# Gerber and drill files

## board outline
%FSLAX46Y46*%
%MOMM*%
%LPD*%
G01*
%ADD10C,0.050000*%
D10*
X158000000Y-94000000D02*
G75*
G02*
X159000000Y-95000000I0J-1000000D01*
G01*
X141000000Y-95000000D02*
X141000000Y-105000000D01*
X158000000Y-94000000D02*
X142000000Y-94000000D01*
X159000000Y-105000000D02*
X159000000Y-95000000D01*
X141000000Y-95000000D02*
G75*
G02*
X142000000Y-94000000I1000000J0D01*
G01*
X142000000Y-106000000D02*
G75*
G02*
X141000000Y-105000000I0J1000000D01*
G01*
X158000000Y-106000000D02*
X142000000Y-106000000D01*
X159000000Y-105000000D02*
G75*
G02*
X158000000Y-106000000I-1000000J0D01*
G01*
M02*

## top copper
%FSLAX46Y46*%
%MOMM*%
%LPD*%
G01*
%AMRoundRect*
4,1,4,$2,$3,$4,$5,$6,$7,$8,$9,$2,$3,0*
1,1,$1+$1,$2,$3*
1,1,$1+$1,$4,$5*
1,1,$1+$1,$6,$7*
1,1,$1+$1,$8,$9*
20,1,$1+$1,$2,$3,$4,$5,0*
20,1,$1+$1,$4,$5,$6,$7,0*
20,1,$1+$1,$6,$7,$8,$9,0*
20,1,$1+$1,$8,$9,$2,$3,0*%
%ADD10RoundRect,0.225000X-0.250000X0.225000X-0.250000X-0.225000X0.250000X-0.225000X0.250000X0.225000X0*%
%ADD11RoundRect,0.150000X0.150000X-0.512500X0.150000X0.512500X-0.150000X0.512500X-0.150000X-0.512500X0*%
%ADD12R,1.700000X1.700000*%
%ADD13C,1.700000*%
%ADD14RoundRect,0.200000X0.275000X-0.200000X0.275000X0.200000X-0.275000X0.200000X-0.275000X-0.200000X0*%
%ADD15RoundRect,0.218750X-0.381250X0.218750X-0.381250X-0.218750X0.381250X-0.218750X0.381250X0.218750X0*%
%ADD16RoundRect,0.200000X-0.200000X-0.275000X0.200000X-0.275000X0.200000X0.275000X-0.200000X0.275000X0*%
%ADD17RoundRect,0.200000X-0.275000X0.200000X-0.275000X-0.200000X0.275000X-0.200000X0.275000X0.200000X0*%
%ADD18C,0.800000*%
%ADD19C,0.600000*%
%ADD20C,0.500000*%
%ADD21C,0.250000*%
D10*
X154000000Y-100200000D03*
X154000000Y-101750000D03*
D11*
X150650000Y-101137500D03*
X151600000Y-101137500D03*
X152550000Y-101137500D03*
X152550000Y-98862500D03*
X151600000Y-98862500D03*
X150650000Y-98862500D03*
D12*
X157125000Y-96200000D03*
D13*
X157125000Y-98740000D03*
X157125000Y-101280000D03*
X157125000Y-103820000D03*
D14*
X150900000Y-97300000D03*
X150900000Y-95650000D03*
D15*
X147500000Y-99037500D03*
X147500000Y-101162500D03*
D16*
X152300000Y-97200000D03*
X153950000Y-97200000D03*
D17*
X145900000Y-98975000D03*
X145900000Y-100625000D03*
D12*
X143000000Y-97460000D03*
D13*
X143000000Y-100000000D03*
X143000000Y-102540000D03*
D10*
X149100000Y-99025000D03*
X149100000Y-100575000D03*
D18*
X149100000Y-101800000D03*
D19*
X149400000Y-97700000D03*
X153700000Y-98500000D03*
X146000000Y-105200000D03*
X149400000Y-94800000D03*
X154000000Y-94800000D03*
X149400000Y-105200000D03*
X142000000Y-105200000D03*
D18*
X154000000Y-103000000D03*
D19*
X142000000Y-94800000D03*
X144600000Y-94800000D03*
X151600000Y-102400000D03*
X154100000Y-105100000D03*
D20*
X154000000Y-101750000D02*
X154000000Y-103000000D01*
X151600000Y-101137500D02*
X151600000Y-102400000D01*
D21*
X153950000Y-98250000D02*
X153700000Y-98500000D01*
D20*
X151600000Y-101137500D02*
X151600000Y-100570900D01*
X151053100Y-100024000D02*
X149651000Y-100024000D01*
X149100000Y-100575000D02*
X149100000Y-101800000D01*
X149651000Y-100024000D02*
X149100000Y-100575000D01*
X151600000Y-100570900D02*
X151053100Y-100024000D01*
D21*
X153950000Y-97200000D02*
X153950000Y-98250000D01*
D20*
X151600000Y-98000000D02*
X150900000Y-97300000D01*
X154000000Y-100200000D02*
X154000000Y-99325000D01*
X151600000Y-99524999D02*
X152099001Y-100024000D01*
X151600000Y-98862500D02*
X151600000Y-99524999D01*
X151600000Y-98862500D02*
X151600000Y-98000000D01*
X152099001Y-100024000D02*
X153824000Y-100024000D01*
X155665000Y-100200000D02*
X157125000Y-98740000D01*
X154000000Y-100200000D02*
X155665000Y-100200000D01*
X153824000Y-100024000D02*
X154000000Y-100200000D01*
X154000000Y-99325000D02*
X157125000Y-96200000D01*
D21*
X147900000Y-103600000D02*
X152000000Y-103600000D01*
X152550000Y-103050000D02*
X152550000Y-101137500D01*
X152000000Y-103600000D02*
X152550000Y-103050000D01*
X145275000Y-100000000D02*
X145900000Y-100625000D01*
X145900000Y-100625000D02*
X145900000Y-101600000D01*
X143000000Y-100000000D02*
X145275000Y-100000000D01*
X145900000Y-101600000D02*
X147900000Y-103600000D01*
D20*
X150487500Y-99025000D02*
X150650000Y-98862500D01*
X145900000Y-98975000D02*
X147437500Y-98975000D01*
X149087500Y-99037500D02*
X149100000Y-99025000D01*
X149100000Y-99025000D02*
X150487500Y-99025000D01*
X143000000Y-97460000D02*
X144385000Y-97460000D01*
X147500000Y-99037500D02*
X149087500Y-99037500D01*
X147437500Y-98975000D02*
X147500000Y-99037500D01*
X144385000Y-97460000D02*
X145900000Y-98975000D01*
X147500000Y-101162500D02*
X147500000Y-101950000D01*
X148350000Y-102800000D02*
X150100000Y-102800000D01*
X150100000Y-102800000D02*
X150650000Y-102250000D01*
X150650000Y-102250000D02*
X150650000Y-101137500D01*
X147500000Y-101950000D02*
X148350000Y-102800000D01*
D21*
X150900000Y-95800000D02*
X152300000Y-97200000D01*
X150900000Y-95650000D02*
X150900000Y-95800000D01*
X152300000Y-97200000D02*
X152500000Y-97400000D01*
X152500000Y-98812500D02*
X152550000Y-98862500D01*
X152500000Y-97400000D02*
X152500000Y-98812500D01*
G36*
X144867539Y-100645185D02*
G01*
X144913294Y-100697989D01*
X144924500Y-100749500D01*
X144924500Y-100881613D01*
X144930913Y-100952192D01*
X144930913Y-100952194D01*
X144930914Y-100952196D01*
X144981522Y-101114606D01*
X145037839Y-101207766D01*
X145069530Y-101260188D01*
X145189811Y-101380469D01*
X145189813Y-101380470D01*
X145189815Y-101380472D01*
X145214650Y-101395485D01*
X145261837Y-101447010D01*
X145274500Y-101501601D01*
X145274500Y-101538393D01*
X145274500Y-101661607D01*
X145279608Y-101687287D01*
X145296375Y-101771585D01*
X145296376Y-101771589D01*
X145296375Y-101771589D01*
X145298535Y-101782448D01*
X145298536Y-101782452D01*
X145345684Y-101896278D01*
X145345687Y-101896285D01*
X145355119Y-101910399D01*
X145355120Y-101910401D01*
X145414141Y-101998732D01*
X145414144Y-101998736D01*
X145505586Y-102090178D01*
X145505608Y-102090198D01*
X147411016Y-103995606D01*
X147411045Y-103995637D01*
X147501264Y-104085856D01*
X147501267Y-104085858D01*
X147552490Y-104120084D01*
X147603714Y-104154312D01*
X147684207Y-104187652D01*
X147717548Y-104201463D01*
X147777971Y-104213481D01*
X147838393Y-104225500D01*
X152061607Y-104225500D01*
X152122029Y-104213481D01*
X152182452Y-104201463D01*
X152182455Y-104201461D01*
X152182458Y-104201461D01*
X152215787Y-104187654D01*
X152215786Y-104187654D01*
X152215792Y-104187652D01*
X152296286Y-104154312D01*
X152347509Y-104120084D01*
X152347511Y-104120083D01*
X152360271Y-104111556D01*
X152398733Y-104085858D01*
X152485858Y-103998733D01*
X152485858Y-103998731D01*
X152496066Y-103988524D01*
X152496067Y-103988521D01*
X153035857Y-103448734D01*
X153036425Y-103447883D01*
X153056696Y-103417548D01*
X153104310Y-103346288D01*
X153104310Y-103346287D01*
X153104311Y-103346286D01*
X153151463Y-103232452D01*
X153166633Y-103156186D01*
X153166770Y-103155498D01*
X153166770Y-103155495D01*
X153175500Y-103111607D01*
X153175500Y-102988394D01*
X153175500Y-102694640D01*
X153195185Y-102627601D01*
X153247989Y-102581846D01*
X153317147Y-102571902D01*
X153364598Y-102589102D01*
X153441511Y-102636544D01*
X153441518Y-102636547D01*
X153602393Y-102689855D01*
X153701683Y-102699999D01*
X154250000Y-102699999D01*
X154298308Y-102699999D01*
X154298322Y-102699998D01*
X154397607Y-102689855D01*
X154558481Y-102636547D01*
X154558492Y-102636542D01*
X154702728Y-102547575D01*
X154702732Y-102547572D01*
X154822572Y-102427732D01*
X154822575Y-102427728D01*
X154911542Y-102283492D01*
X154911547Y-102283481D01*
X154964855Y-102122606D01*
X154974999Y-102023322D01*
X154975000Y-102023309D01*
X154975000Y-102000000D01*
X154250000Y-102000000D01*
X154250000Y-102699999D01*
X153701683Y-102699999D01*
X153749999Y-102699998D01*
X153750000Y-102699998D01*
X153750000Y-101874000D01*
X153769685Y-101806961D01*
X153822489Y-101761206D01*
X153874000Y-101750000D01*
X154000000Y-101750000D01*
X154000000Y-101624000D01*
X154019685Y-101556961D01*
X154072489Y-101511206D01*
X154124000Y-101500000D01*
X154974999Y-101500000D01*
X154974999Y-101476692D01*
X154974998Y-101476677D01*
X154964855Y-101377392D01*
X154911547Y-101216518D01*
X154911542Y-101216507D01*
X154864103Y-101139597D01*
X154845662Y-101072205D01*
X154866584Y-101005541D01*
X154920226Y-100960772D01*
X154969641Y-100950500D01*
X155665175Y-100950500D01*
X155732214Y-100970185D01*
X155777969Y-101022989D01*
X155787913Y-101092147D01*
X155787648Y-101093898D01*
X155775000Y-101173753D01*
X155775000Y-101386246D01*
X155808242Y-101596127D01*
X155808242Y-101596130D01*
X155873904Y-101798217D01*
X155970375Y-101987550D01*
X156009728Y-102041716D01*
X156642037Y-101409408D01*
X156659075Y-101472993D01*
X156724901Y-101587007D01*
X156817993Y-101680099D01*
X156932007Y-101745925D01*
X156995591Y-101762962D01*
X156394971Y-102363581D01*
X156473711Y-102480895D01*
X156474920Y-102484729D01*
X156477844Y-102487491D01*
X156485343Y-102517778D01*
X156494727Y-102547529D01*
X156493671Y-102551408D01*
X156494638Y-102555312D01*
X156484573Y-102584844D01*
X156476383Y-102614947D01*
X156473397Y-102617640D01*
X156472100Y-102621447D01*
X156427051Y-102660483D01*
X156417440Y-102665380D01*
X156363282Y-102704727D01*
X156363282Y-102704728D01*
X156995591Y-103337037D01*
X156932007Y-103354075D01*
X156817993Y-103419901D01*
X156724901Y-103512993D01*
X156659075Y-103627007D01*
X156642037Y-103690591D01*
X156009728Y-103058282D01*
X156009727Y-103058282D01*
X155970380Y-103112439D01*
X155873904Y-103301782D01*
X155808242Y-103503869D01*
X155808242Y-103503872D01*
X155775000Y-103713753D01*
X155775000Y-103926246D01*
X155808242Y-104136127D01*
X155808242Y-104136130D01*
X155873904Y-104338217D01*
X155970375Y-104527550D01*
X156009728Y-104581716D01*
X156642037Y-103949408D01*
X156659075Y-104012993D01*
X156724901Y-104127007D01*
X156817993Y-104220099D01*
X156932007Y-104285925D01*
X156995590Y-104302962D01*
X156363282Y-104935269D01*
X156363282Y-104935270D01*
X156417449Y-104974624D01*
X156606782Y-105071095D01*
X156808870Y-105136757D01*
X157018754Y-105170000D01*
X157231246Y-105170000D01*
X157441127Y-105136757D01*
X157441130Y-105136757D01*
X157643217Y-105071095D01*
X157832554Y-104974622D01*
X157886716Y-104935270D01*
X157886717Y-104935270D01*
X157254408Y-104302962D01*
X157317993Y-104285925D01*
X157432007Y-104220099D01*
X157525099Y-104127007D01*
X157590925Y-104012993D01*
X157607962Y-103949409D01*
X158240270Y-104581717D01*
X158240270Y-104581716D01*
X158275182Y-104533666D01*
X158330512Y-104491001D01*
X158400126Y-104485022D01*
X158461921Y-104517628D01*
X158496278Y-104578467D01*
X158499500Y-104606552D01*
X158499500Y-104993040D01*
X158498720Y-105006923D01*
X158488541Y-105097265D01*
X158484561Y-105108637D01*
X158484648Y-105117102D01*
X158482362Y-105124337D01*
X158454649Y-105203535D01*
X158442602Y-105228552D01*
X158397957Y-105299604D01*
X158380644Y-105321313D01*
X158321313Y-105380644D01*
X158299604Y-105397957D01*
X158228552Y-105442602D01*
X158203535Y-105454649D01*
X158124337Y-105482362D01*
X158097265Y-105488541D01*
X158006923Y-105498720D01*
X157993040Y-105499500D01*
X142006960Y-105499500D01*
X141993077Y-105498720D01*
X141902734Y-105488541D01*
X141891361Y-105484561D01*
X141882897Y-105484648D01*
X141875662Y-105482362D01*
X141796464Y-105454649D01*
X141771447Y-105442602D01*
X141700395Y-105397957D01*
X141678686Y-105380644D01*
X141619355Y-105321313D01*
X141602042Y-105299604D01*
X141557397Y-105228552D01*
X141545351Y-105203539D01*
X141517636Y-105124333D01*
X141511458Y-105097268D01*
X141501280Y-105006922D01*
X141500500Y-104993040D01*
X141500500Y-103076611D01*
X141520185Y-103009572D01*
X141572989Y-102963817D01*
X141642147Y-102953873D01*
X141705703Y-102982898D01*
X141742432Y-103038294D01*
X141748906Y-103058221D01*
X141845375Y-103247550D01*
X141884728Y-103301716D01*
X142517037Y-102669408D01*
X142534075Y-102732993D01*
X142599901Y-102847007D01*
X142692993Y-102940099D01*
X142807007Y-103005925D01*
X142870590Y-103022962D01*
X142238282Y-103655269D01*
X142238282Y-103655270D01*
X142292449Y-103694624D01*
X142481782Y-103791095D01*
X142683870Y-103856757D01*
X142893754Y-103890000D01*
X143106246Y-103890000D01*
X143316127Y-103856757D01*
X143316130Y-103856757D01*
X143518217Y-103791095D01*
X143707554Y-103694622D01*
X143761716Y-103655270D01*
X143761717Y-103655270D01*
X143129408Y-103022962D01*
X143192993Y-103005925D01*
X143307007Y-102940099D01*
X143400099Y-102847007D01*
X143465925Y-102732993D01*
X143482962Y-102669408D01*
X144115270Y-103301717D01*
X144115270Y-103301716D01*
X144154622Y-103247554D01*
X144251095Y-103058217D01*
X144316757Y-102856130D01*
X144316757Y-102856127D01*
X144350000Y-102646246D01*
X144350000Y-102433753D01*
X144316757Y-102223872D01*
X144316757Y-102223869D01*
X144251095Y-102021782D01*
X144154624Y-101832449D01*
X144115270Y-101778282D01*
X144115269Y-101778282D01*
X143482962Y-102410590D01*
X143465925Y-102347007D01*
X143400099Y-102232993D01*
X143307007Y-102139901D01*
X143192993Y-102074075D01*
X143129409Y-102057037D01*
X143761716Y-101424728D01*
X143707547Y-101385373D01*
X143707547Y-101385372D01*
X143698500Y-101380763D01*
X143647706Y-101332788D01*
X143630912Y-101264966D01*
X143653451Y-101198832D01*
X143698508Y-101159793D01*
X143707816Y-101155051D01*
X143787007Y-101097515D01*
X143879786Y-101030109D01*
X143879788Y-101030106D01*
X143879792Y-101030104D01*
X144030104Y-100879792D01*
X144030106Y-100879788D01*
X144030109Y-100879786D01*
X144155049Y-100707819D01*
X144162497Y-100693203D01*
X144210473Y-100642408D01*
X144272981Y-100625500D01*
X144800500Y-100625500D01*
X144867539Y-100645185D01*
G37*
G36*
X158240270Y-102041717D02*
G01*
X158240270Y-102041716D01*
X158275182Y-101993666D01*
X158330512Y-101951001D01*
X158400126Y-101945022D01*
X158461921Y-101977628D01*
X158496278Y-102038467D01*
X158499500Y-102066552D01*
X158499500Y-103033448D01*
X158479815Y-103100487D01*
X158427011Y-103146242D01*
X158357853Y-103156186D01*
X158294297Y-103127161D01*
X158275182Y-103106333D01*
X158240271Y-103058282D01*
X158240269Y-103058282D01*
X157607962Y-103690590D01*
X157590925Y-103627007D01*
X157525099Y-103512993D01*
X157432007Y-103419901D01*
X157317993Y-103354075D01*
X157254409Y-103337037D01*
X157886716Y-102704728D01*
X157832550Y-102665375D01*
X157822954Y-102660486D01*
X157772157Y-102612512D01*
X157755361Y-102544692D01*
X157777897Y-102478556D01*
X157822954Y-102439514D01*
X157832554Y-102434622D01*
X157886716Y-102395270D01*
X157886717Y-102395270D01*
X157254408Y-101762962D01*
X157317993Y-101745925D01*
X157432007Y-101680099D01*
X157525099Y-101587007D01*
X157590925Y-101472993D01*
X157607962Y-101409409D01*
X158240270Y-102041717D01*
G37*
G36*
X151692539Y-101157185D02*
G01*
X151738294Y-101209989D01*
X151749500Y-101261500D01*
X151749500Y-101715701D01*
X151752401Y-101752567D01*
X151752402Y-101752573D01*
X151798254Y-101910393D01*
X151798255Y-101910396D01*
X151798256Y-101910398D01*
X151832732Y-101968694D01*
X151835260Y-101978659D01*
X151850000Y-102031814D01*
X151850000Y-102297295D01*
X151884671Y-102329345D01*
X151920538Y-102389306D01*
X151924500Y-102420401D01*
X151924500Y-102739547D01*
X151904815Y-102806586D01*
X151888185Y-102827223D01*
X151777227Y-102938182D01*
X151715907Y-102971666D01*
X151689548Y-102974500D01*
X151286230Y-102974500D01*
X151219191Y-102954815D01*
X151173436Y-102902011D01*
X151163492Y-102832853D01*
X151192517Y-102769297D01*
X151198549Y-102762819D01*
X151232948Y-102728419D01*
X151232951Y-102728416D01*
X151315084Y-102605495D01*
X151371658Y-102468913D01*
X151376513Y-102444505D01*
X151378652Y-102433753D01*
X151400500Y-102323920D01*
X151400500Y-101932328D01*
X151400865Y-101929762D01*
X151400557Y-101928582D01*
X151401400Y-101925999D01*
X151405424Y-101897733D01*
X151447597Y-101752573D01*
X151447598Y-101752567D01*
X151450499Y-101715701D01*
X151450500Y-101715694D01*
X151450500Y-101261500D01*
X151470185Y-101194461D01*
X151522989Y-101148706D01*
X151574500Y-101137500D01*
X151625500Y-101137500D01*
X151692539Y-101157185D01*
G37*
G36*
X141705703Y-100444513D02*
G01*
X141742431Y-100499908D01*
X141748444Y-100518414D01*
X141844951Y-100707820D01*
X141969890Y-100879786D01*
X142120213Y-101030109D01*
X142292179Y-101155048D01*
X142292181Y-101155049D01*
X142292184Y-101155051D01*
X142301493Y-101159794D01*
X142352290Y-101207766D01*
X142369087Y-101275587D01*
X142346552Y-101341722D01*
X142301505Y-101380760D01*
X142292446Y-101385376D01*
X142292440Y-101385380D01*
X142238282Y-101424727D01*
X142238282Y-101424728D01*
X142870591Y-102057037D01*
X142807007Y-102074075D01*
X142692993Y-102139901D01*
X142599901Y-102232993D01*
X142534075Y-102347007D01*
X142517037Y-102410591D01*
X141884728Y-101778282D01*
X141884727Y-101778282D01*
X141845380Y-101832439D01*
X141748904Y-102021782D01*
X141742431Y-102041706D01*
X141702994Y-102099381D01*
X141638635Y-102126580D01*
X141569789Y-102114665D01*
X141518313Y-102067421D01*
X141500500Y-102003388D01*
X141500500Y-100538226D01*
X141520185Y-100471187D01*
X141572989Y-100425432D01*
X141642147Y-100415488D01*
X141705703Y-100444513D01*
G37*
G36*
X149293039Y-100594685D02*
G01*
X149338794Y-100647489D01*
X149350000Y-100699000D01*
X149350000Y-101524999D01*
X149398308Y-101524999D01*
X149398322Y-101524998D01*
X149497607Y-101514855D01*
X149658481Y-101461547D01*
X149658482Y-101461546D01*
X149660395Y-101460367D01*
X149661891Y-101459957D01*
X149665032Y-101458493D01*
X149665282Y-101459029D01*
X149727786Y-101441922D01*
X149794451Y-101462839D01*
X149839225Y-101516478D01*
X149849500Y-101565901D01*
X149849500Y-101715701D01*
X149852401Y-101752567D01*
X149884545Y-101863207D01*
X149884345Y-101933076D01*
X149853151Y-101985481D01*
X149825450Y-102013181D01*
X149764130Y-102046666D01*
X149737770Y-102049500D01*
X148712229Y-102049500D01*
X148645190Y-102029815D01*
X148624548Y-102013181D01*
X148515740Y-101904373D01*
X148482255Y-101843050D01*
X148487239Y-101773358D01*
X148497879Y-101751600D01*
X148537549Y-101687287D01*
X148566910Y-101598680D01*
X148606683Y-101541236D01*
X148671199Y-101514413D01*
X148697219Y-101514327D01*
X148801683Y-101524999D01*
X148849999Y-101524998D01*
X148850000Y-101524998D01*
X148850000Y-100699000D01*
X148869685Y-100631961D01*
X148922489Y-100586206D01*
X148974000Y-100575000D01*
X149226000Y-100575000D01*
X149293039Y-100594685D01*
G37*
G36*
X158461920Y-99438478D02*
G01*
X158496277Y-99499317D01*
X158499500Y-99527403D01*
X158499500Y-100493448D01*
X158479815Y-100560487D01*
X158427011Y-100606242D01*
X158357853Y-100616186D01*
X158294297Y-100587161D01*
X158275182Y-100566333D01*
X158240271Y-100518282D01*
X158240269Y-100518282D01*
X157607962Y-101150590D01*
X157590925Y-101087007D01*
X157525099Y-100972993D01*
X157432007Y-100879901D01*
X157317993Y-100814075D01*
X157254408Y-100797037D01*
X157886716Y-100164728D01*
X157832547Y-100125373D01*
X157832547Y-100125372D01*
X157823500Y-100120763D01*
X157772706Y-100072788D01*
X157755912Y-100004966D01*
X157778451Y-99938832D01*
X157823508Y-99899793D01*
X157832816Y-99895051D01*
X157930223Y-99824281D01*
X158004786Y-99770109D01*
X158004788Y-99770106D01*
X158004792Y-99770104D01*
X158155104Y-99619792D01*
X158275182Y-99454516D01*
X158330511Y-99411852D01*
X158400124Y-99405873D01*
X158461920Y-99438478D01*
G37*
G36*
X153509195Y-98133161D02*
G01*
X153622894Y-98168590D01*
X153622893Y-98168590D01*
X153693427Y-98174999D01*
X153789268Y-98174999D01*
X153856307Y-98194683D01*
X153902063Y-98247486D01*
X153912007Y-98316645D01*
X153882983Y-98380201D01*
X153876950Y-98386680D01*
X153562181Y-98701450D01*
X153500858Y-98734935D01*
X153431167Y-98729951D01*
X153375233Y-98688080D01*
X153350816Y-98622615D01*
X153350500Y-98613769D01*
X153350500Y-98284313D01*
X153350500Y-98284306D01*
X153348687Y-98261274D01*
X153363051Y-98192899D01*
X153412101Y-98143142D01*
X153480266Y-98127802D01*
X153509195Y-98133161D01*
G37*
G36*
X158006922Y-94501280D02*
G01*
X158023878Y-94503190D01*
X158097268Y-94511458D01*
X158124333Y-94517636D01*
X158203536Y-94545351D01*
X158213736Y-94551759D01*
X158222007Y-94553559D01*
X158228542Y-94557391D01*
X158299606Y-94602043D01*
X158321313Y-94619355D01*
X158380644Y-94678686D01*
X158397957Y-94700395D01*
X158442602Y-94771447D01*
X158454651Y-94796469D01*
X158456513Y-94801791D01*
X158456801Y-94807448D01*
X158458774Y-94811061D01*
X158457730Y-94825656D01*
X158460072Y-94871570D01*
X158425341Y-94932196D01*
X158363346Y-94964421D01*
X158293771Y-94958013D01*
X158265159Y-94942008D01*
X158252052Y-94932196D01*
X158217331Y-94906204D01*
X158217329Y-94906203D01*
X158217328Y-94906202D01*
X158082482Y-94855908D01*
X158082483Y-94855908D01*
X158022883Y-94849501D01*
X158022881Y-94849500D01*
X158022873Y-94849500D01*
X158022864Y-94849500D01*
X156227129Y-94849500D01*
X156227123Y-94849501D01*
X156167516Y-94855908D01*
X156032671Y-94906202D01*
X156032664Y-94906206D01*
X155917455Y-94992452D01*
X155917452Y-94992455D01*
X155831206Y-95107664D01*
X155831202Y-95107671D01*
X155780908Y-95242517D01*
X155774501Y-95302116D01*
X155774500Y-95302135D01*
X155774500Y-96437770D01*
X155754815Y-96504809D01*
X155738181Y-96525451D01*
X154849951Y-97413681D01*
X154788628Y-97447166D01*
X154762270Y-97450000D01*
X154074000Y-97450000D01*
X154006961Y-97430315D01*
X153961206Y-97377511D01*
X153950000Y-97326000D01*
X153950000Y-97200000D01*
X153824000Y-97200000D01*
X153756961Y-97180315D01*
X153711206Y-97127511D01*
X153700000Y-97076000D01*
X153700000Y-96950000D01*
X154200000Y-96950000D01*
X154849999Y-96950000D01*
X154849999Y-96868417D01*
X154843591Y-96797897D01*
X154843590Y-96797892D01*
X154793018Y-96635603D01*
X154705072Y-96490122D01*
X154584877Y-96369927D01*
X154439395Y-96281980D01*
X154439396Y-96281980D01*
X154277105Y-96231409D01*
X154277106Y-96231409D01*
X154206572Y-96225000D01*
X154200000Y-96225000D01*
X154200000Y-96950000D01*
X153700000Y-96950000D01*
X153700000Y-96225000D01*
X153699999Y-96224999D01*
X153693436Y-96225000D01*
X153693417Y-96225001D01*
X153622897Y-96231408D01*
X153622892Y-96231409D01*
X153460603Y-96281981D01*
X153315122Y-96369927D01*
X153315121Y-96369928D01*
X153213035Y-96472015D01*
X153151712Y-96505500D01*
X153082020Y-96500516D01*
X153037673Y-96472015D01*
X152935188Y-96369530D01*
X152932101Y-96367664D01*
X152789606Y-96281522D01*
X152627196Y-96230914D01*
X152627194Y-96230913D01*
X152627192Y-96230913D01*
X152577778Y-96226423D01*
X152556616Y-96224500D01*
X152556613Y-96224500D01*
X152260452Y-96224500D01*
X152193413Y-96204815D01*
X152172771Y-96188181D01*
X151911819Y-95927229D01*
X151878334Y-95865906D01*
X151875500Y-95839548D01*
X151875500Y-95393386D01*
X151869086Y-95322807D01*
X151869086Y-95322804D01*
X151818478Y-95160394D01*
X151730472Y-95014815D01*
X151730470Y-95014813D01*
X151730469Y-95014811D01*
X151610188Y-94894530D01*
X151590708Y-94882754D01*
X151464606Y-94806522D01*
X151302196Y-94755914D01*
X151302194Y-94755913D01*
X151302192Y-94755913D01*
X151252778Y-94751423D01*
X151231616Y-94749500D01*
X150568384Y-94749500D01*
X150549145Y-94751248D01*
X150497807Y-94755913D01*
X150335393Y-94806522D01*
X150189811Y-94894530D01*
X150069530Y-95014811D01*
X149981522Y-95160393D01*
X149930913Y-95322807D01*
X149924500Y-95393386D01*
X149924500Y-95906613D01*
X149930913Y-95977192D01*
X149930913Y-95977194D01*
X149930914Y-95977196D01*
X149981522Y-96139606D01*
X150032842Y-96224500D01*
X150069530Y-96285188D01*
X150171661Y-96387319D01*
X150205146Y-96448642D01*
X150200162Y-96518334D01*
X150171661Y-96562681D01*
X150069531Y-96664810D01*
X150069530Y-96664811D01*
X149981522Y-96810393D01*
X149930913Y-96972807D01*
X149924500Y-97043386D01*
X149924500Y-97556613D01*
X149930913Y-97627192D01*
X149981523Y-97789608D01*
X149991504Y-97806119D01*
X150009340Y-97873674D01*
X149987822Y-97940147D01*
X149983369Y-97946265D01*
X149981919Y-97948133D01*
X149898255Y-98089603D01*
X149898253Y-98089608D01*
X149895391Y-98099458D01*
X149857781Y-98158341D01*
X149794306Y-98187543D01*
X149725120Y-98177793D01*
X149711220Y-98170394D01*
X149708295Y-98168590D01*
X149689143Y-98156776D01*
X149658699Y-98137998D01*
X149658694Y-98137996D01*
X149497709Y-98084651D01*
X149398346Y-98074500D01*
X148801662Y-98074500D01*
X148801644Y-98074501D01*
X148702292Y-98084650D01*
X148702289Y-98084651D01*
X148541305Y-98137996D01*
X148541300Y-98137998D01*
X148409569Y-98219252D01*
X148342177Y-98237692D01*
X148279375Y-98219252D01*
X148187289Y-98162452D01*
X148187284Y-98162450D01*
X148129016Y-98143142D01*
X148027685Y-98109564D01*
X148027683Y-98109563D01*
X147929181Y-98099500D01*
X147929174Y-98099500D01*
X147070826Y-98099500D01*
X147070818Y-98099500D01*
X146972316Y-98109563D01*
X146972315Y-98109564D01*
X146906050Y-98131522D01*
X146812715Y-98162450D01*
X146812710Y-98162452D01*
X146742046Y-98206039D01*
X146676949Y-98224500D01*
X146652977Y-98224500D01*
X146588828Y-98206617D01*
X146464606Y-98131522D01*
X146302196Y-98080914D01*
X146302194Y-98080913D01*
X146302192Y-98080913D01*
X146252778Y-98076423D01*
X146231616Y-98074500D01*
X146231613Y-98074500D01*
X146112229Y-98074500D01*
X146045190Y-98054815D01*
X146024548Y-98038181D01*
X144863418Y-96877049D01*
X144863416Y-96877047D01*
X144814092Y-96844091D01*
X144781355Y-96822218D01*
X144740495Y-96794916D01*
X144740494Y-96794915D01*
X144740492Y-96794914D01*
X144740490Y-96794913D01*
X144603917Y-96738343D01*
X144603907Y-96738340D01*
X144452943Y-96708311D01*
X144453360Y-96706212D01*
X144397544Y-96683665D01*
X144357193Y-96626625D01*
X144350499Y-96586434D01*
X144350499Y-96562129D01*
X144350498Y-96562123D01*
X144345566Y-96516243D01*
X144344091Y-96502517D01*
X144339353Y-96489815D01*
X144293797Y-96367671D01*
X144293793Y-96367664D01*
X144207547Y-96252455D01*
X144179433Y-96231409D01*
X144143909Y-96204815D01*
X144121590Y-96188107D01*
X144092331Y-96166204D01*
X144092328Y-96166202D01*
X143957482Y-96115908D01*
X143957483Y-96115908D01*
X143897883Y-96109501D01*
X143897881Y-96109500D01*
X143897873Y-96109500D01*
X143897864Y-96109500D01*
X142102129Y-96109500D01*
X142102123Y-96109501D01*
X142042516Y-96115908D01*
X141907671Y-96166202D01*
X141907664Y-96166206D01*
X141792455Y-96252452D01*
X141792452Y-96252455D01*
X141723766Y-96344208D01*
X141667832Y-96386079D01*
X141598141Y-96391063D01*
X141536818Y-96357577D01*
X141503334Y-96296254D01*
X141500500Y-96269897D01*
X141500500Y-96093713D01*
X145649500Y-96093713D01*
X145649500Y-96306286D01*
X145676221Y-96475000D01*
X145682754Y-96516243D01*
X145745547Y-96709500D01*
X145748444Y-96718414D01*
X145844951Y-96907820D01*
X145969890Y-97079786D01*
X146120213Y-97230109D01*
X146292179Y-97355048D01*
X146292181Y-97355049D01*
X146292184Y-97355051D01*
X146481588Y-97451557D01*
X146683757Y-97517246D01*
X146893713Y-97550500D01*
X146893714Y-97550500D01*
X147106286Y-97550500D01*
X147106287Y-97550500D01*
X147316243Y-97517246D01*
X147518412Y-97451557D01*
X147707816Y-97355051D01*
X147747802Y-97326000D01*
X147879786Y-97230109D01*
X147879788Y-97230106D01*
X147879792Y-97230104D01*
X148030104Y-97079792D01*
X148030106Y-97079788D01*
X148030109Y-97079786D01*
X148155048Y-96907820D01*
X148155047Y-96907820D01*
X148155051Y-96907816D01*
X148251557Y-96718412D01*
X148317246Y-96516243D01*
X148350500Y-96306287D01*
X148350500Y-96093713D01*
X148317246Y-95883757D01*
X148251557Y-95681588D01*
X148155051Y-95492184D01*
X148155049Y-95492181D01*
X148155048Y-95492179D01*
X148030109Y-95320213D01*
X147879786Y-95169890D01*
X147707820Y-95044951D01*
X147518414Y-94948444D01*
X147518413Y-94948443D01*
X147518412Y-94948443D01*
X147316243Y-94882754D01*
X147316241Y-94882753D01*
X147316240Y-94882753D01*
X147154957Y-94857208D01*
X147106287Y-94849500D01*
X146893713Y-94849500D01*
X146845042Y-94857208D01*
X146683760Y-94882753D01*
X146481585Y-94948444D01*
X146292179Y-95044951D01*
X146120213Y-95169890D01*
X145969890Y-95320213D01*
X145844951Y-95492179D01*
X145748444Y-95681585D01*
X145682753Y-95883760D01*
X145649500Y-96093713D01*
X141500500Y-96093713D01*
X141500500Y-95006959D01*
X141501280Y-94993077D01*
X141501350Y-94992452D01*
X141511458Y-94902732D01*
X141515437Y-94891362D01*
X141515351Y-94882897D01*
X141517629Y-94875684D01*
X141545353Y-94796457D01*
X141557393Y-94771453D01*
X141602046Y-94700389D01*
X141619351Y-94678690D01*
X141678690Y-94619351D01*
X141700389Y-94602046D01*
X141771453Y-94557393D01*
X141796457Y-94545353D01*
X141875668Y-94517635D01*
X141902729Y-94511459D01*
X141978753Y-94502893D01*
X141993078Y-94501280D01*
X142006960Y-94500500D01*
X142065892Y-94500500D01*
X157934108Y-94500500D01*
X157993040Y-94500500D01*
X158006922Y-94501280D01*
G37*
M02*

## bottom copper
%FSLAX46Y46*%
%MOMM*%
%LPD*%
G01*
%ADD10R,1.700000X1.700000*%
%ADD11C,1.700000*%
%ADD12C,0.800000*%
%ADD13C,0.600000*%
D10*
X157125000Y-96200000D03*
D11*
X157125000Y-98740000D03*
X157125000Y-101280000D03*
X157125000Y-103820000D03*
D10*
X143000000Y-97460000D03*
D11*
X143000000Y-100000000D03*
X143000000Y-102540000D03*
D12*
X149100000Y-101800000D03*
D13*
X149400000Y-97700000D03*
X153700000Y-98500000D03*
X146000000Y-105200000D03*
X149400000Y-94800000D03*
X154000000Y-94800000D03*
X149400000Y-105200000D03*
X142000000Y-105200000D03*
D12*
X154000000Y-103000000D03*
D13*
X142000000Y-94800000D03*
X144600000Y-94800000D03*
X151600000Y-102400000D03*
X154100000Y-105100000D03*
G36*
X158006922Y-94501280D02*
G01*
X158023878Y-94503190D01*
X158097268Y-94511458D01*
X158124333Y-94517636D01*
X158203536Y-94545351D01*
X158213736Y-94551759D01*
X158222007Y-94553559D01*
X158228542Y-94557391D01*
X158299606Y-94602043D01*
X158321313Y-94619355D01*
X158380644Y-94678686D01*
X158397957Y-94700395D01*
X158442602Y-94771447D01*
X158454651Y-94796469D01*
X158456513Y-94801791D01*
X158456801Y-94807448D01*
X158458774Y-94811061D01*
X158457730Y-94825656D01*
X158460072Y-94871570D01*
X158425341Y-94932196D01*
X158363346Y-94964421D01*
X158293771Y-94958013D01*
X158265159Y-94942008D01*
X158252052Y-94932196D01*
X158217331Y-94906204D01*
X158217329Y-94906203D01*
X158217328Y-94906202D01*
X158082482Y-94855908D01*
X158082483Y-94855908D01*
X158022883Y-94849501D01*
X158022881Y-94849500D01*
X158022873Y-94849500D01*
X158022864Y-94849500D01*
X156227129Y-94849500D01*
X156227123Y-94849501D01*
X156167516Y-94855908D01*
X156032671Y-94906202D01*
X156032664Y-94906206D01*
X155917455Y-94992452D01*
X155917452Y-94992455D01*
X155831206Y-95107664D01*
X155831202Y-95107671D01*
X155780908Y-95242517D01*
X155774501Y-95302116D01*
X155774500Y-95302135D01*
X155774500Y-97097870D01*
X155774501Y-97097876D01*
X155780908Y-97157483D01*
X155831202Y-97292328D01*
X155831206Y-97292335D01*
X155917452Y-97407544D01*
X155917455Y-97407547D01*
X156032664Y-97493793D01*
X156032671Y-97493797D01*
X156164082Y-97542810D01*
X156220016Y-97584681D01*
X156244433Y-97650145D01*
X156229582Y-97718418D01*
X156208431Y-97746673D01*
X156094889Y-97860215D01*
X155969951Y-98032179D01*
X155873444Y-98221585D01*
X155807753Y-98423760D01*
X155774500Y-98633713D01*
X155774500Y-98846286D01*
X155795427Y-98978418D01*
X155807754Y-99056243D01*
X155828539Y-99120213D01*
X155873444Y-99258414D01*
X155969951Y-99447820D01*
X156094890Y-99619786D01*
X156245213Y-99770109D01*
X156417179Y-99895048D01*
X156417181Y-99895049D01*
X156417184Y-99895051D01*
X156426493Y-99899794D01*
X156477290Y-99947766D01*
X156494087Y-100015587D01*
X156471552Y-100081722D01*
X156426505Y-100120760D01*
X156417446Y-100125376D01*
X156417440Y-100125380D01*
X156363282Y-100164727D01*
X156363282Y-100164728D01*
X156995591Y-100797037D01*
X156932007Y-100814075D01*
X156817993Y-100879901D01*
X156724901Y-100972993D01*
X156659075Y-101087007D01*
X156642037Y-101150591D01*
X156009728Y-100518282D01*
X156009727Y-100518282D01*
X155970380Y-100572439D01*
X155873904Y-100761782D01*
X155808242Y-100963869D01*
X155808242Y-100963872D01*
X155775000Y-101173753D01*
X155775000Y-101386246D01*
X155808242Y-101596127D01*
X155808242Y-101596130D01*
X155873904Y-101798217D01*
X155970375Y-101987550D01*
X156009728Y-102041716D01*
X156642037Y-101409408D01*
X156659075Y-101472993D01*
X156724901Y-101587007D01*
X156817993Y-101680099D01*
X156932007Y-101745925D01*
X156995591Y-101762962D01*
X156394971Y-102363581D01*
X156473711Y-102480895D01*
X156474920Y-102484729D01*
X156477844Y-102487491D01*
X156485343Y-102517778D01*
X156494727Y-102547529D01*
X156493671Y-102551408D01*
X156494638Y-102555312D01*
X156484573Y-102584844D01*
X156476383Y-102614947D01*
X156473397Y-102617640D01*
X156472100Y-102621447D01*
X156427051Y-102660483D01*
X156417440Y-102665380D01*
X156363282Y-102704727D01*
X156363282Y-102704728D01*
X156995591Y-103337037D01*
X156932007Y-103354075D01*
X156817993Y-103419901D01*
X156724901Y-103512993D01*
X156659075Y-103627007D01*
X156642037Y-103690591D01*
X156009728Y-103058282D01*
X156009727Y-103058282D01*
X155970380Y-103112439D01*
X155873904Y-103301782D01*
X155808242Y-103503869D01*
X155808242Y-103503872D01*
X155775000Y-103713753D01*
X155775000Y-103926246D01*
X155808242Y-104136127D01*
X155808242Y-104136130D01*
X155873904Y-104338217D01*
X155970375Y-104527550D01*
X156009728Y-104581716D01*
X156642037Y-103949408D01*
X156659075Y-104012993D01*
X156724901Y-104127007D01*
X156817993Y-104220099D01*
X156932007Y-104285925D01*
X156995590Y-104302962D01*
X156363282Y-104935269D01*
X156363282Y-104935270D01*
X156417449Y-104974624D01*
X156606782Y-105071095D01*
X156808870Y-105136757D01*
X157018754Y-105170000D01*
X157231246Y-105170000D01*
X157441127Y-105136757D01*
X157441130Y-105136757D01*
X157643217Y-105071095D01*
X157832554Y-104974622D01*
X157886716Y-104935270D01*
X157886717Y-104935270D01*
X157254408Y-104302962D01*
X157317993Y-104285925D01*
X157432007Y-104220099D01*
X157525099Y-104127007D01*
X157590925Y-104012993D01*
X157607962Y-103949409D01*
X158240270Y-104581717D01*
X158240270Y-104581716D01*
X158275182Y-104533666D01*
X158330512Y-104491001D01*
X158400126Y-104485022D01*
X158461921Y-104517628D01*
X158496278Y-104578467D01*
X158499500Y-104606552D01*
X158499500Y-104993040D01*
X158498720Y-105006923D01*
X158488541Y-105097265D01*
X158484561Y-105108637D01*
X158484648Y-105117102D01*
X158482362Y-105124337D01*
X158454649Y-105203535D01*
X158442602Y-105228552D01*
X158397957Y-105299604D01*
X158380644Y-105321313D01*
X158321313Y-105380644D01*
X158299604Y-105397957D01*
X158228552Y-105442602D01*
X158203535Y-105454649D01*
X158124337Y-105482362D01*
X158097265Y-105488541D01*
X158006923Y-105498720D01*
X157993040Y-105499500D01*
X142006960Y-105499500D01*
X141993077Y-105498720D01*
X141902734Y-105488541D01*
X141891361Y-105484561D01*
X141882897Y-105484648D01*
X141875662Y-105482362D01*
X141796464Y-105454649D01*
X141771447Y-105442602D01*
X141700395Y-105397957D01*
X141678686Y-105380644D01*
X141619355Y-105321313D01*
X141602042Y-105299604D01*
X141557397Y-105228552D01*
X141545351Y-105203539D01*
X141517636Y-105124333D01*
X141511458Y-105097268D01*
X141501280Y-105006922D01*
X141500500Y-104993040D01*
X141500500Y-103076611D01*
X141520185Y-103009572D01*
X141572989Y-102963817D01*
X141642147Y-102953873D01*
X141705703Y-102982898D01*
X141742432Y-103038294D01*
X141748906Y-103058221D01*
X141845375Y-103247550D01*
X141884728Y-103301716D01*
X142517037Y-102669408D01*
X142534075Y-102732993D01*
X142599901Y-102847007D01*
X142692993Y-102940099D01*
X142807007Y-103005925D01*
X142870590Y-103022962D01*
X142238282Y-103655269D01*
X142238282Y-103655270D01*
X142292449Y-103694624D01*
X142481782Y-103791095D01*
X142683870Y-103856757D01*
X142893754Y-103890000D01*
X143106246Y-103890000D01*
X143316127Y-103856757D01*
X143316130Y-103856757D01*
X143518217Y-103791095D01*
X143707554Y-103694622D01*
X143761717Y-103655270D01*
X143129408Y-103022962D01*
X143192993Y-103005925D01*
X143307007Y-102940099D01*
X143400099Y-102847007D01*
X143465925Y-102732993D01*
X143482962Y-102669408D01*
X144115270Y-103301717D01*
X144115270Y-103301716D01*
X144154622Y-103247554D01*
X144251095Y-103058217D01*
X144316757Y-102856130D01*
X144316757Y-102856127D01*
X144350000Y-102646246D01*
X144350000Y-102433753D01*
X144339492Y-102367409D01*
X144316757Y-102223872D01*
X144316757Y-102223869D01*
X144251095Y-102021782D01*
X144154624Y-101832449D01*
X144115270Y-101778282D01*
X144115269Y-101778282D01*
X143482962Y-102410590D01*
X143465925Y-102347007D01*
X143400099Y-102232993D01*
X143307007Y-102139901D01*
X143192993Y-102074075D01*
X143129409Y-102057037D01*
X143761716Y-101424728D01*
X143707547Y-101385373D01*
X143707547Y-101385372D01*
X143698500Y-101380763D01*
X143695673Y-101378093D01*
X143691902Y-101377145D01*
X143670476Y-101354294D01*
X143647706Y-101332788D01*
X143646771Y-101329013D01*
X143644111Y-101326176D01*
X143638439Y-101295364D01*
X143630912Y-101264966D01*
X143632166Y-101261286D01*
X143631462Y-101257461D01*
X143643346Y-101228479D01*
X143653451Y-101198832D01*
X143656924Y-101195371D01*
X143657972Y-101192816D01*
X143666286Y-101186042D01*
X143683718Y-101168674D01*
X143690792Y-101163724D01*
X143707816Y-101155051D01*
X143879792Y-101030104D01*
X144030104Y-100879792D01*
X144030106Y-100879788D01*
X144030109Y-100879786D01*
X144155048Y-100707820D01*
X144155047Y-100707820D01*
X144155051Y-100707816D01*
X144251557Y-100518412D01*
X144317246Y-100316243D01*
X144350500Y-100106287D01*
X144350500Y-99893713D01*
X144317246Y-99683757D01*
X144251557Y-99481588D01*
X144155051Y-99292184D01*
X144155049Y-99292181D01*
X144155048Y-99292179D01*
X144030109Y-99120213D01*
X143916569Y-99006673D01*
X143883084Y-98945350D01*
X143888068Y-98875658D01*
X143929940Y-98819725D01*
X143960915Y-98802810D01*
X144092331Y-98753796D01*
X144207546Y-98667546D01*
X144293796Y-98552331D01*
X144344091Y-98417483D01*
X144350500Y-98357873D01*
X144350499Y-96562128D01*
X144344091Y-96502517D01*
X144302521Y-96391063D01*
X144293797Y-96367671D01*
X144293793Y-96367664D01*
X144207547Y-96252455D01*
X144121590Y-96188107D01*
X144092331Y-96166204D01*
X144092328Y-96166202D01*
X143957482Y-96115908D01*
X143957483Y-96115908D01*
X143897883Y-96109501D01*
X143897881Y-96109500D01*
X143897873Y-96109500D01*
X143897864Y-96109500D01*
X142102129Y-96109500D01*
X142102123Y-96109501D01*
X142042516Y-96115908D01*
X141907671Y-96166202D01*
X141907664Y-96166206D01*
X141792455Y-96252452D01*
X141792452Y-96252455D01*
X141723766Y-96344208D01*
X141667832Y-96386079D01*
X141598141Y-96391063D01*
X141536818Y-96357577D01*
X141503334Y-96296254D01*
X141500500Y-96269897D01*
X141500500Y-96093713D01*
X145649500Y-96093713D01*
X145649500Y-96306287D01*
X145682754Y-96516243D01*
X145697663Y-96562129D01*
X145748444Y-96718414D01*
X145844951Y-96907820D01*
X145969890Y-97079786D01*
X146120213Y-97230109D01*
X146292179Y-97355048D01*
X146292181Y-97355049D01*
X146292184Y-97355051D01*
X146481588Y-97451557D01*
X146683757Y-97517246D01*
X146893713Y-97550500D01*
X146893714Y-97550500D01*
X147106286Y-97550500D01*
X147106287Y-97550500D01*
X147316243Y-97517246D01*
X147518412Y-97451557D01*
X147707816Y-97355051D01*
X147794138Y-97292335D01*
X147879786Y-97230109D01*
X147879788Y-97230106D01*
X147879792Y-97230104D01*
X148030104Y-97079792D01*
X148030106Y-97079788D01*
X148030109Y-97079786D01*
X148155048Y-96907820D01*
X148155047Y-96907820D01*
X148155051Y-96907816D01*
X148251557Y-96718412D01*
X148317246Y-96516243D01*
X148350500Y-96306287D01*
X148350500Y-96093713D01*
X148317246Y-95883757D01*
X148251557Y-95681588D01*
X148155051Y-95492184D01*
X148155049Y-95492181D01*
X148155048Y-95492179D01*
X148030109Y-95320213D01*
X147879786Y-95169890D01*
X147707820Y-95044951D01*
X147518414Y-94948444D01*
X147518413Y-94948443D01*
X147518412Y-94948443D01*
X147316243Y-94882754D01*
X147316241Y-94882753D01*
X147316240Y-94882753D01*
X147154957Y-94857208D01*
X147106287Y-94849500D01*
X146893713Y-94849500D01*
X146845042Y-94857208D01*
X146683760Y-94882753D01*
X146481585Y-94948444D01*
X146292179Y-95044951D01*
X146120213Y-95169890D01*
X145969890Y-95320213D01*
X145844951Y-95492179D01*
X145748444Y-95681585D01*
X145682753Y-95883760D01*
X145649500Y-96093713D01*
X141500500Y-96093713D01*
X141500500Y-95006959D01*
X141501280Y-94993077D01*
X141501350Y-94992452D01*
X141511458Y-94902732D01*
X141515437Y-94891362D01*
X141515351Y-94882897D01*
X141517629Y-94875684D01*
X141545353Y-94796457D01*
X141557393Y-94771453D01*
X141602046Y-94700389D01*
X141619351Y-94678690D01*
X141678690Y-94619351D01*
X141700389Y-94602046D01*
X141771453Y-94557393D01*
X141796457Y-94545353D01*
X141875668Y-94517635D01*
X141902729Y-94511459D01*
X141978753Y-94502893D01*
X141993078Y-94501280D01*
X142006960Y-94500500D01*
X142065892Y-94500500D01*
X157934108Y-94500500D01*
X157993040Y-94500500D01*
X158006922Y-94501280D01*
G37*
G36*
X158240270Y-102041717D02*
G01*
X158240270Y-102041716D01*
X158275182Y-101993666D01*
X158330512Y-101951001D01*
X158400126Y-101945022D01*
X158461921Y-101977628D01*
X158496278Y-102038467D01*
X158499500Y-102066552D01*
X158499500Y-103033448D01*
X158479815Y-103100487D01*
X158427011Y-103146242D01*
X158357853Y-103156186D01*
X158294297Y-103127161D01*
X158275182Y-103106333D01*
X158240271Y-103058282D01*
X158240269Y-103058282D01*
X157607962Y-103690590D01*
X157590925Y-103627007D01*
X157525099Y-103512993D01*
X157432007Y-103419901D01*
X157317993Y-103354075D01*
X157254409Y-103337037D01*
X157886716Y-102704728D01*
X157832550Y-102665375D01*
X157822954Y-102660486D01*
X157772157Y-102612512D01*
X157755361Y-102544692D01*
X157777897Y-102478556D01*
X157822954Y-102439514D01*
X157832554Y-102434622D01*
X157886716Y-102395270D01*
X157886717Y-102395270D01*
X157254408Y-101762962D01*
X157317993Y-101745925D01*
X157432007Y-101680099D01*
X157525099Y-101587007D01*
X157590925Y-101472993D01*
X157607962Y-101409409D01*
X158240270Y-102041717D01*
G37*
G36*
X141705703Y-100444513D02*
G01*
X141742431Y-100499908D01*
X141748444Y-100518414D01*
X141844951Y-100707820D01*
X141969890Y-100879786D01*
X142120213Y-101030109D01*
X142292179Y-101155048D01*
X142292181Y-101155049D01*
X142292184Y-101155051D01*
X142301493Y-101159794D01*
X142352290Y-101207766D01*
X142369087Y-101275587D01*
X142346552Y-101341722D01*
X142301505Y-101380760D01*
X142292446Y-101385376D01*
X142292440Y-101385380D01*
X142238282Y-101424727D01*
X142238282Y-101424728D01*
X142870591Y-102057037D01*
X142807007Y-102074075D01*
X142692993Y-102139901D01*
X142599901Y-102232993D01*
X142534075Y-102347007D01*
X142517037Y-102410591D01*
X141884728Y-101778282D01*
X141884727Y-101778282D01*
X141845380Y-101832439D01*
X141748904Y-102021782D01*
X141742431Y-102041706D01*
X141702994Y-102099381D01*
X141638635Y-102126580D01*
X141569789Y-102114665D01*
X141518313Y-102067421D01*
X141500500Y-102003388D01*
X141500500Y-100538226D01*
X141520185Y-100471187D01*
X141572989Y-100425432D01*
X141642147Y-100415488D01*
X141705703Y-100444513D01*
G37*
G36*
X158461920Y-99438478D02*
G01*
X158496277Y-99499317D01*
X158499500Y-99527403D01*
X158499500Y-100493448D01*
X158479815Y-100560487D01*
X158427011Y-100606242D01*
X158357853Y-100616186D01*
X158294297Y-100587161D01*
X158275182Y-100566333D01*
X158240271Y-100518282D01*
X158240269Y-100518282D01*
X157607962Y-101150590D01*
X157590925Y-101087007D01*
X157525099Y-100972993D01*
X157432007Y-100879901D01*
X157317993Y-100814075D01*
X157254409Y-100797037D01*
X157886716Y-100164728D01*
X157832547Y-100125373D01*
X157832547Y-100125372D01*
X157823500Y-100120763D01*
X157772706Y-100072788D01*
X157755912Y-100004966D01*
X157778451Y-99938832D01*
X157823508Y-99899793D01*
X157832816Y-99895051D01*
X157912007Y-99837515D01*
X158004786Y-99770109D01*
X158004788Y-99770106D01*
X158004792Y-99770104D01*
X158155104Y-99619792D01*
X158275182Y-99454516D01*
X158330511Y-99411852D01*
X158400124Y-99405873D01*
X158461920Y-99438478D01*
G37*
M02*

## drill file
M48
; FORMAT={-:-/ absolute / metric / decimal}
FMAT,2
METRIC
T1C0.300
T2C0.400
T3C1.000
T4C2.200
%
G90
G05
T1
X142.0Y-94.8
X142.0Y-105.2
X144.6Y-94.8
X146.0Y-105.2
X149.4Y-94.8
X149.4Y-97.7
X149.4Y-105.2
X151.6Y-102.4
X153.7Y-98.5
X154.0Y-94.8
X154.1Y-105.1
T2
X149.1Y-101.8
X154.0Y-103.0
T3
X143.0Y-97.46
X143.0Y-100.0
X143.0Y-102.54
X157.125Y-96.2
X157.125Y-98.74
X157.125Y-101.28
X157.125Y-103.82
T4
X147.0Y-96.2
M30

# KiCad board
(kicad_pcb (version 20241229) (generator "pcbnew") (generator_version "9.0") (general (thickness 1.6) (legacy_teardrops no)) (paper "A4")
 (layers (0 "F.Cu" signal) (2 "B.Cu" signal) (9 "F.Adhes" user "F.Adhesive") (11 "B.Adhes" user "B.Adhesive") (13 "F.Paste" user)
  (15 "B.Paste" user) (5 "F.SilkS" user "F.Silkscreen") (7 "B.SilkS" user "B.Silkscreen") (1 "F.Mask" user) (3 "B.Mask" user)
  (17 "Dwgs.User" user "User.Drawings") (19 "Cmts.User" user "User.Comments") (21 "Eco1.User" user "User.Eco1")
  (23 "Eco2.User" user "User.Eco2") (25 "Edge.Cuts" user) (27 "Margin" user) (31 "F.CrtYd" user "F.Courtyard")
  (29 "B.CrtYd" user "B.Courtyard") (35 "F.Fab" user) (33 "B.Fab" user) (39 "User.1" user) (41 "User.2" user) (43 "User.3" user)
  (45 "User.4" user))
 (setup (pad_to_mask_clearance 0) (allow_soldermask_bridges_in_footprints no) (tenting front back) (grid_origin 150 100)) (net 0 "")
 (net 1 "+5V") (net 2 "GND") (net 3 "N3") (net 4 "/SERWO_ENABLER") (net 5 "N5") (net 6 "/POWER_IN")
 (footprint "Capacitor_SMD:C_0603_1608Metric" (layer "F.Cu") (at 154 100.975 -90)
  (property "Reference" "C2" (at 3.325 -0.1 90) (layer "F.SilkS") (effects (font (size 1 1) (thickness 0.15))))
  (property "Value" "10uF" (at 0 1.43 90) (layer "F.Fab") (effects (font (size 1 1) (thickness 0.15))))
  (pad "1" smd roundrect (at -0.775 0 270) (size 0.9 0.95) (layers "F.Cu" "F.Mask" "F.Paste") (roundrect_rratio 0.25) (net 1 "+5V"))
  (pad "2" smd roundrect (at 0.775 0 270) (size 0.9 0.95) (layers "F.Cu" "F.Mask" "F.Paste") (roundrect_rratio 0.25) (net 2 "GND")))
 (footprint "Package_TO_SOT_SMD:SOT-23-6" (layer "F.Cu") (at 151.6 100 90)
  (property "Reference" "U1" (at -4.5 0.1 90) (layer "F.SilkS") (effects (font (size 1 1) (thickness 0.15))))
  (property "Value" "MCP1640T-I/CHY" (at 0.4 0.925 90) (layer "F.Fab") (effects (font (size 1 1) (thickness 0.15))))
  (pad "1" smd roundrect (at -1.1375 -0.95 90) (size 1.325 0.6) (layers "F.Cu" "F.Mask" "F.Paste") (roundrect_rratio 0.25) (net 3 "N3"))
  (pad "2" smd roundrect (at -1.1375 0 90) (size 1.325 0.6) (layers "F.Cu" "F.Mask" "F.Paste") (roundrect_rratio 0.25) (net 2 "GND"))
  (pad "3" smd roundrect (at -1.1375 0.95 90) (size 1.325 0.6) (layers "F.Cu" "F.Mask" "F.Paste") (roundrect_rratio 0.25)
   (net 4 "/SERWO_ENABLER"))
  (pad "4" smd roundrect (at 1.1375 0.95 90) (size 1.325 0.6) (layers "F.Cu" "F.Mask" "F.Paste") (roundrect_rratio 0.25) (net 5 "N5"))
  (pad "5" smd roundrect (at 1.1375 0 90) (size 1.325 0.6) (layers "F.Cu" "F.Mask" "F.Paste") (roundrect_rratio 0.25) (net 1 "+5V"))
  (pad "6" smd roundrect (at 1.1375 -0.95 90) (size 1.325 0.6) (layers "F.Cu" "F.Mask" "F.Paste") (roundrect_rratio 0.25)
   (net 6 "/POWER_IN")))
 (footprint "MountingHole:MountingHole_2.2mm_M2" (layer "F.Cu") (at 147 96.2)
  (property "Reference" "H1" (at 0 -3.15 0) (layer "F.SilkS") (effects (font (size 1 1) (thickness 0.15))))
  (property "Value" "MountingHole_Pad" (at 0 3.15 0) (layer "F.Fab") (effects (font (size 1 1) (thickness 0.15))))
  (pad "" np_thru_hole circle (at 0 0) (size 2.2 2.2) (drill 2.2) (layers "*.Cu" "*.Mask")))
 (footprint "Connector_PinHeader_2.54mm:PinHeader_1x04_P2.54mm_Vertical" (layer "F.Cu") (at 157.125 96.2)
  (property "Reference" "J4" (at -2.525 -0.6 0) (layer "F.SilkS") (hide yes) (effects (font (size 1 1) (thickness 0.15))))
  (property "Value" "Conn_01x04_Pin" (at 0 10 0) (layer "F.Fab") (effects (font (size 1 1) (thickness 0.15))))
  (pad "1" thru_hole rect (at 0 0) (size 1.7 1.7) (drill 1) (layers "*.Cu" "*.Mask") (remove_unused_layers no) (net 1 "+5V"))
  (pad "2" thru_hole circle (at 0 2.54) (size 1.7 1.7) (drill 1) (layers "*.Cu" "*.Mask") (remove_unused_layers no) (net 1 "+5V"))
  (pad "3" thru_hole circle (at 0 5.08) (size 1.7 1.7) (drill 1) (layers "*.Cu" "*.Mask") (remove_unused_layers no) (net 2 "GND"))
  (pad "4" thru_hole circle (at 0 7.62) (size 1.7 1.7) (drill 1) (layers "*.Cu" "*.Mask") (remove_unused_layers no) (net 2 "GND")))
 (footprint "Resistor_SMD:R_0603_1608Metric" (layer "F.Cu") (at 150.9 96.475 90)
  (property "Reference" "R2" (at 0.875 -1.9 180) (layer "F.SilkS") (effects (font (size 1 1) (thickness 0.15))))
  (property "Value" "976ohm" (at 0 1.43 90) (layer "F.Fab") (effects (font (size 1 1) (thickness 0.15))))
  (pad "1" smd roundrect (at -0.825 0 90) (size 0.8 0.95) (layers "F.Cu" "F.Mask" "F.Paste") (roundrect_rratio 0.25) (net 1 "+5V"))
  (pad "2" smd roundrect (at 0.825 0 90) (size 0.8 0.95) (layers "F.Cu" "F.Mask" "F.Paste") (roundrect_rratio 0.25) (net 5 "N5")))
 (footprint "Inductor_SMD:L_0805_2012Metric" (layer "F.Cu") (at 147.5 100.1 -90)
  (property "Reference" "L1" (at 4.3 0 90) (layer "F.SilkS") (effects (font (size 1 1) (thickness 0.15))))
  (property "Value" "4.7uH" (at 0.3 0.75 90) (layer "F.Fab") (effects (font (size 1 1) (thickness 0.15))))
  (pad "1" smd roundrect (at -1.0625 0 270) (size 0.875 1.2) (layers "F.Cu" "F.Mask" "F.Paste") (roundrect_rratio 0.25) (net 6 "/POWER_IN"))
  (pad "2" smd roundrect (at 1.0625 0 270) (size 0.875 1.2) (layers "F.Cu" "F.Mask" "F.Paste") (roundrect_rratio 0.25) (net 3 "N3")))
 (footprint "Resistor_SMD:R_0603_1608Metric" (layer "F.Cu") (at 153.125 97.2)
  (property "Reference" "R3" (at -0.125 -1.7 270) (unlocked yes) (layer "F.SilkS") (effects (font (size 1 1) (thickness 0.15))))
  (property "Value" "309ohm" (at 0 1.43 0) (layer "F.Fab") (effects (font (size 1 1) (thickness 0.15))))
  (pad "1" smd roundrect (at -0.825 0) (size 0.8 0.95) (layers "F.Cu" "F.Mask" "F.Paste") (roundrect_rratio 0.25) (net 5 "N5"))
  (pad "2" smd roundrect (at 0.825 0) (size 0.8 0.95) (layers "F.Cu" "F.Mask" "F.Paste") (roundrect_rratio 0.25) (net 2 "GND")))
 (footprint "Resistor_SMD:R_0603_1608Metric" (layer "F.Cu") (at 145.9 99.8 -90)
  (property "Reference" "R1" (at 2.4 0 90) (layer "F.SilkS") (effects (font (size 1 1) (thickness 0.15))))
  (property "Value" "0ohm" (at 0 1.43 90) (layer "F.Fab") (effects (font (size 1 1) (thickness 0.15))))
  (pad "1" smd roundrect (at -0.825 0 270) (size 0.8 0.95) (layers "F.Cu" "F.Mask" "F.Paste") (roundrect_rratio 0.25) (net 6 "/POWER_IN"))
  (pad "2" smd roundrect (at 0.825 0 270) (size 0.8 0.95) (layers "F.Cu" "F.Mask" "F.Paste") (roundrect_rratio 0.25)
   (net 4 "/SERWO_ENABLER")))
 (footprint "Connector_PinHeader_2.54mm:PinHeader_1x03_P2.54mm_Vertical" (layer "F.Cu") (at 143 97.46)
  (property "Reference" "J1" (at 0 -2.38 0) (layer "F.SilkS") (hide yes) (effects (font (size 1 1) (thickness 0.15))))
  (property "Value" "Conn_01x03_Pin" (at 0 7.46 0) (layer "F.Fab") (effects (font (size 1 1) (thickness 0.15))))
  (pad "1" thru_hole rect (at 0 0) (size 1.7 1.7) (drill 1) (layers "*.Cu" "*.Mask") (remove_unused_layers no) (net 6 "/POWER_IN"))
  (pad "2" thru_hole circle (at 0 2.54) (size 1.7 1.7) (drill 1) (layers "*.Cu" "*.Mask") (remove_unused_layers no) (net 4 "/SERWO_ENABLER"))
  (pad "3" thru_hole circle (at 0 5.08) (size 1.7 1.7) (drill 1) (layers "*.Cu" "*.Mask") (remove_unused_layers no) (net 2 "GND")))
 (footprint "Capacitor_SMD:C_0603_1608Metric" (layer "F.Cu") (at 149.1 99.8 -90)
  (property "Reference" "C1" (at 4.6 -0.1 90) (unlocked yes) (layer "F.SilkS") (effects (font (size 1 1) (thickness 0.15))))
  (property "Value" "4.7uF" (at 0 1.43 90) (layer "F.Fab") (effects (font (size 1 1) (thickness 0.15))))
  (pad "1" smd roundrect (at -0.775 0 270) (size 0.9 0.95) (layers "F.Cu" "F.Mask" "F.Paste") (roundrect_rratio 0.25) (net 6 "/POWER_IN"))
  (pad "2" smd roundrect (at 0.775 0 270) (size 0.9 0.95) (layers "F.Cu" "F.Mask" "F.Paste") (roundrect_rratio 0.25) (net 2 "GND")))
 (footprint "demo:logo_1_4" (layer "B.Cu") (at 150 100 180)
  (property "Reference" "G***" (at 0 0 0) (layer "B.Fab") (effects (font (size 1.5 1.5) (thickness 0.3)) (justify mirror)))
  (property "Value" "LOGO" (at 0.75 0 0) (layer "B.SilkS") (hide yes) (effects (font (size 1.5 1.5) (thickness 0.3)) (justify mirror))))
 (gr_arc (start 158 94) (mid 158.707107 94.292893) (end 159 95) (stroke (width 0.05) (type default)) (layer "Edge.Cuts"))
 (gr_line (start 141 95) (end 141 105) (stroke (width 0.05) (type default)) (layer "Edge.Cuts"))
 (gr_line (start 158 94) (end 142 94) (stroke (width 0.05) (type default)) (layer "Edge.Cuts"))
 (gr_line (start 159 105) (end 159 95) (stroke (width 0.05) (type default)) (layer "Edge.Cuts"))
 (gr_arc (start 141 95) (mid 141.292893 94.292893) (end 142 94) (stroke (width 0.05) (type default)) (layer "Edge.Cuts"))
 (gr_arc (start 142 106) (mid 141.292893 105.707107) (end 141 105) (stroke (width 0.05) (type default)) (layer "Edge.Cuts"))
 (gr_line (start 158 106) (end 142 106) (stroke (width 0.05) (type default)) (layer "Edge.Cuts"))
 (gr_arc (start 159 105) (mid 158.707107 105.707107) (end 158 106) (stroke (width 0.05) (type default)) (layer "Edge.Cuts"))
 (segment (start 154 101.75) (end 154 103) (width 0.5) (layer "F.Cu") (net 2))
 (segment (start 151.6 101.1375) (end 151.6 102.4) (width 0.5) (layer "F.Cu") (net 2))
 (segment (start 153.95 98.25) (end 153.7 98.5) (width 0.25) (layer "F.Cu") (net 2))
 (segment (start 151.6 101.1375) (end 151.6 100.5709) (width 0.5) (layer "F.Cu") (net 2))
 (segment (start 151.0531 100.024) (end 149.651 100.024) (width 0.5) (layer "F.Cu") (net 2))
 (segment (start 149.1 100.575) (end 149.1 101.8) (width 0.5) (layer "F.Cu") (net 2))
 (segment (start 149.651 100.024) (end 149.1 100.575) (width 0.5) (layer "F.Cu") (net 2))
 (segment (start 151.6 100.5709) (end 151.0531 100.024) (width 0.5) (layer "F.Cu") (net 2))
 (segment (start 153.95 97.2) (end 153.95 98.25) (width 0.25) (layer "F.Cu") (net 2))
 (via (at 149.1 101.8) (size 0.8) (drill 0.4) (layers "F.Cu" "B.Cu") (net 2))
 (via (at 149.4 97.7) (size 0.6) (drill 0.3) (layers "F.Cu" "B.Cu") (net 2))
 (via (at 153.7 98.5) (size 0.6) (drill 0.3) (layers "F.Cu" "B.Cu") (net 2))
 (via (at 146 105.2) (size 0.6) (drill 0.3) (layers "F.Cu" "B.Cu") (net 2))
 (via (at 149.4 94.8) (size 0.6) (drill 0.3) (layers "F.Cu" "B.Cu") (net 2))
 (via (at 154 94.8) (size 0.6) (drill 0.3) (layers "F.Cu" "B.Cu") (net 2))
 (via (at 149.4 105.2) (size 0.6) (drill 0.3) (layers "F.Cu" "B.Cu") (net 2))
 (via (at 142 105.2) (size 0.6) (drill 0.3) (layers "F.Cu" "B.Cu") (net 2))
 (via (at 154 103) (size 0.8) (drill 0.4) (layers "F.Cu" "B.Cu") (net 2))
 (via (at 142 94.8) (size 0.6) (drill 0.3) (layers "F.Cu" "B.Cu") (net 2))
 (via (at 144.6 94.8) (size 0.6) (drill 0.3) (layers "F.Cu" "B.Cu") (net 2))
 (via (at 151.6 102.4) (size 0.6) (drill 0.3) (layers "F.Cu" "B.Cu") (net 2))
 (via (at 154.1 105.1) (size 0.6) (drill 0.3) (layers "F.Cu" "B.Cu") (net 2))
 (segment (start 151.6 98) (end 150.9 97.3) (width 0.5) (layer "F.Cu") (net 1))
 (segment (start 154 100.2) (end 154 99.325) (width 0.5) (layer "F.Cu") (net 1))
 (segment (start 151.6 99.524999) (end 152.099001 100.024) (width 0.5) (layer "F.Cu") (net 1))
 (segment (start 151.6 98.8625) (end 151.6 99.524999) (width 0.5) (layer "F.Cu") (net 1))
 (segment (start 151.6 98.8625) (end 151.6 98) (width 0.5) (layer "F.Cu") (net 1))
 (segment (start 152.099001 100.024) (end 153.824 100.024) (width 0.5) (layer "F.Cu") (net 1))
 (segment (start 155.665 100.2) (end 157.125 98.74) (width 0.5) (layer "F.Cu") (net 1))
 (segment (start 154 100.2) (end 155.665 100.2) (width 0.5) (layer "F.Cu") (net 1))
 (segment (start 153.824 100.024) (end 154 100.2) (width 0.5) (layer "F.Cu") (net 1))
 (segment (start 154 99.325) (end 157.125 96.2) (width 0.5) (layer "F.Cu") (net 1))
 (segment (start 147.9 103.6) (end 152 103.6) (width 0.25) (layer "F.Cu") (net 4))
 (segment (start 152.55 103.05) (end 152.55 101.1375) (width 0.25) (layer "F.Cu") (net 4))
 (segment (start 152 103.6) (end 152.55 103.05) (width 0.25) (layer "F.Cu") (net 4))
 (segment (start 145.275 100) (end 145.9 100.625) (width 0.25) (layer "F.Cu") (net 4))
 (segment (start 145.9 100.625) (end 145.9 101.6) (width 0.25) (layer "F.Cu") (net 4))
 (segment (start 143 100) (end 145.275 100) (width 0.25) (layer "F.Cu") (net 4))
 (segment (start 145.9 101.6) (end 147.9 103.6) (width 0.25) (layer "F.Cu") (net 4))
 (segment (start 150.4875 99.025) (end 150.65 98.8625) (width 0.5) (layer "F.Cu") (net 6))
 (segment (start 145.9 98.975) (end 147.4375 98.975) (width 0.5) (layer "F.Cu") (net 6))
 (segment (start 149.0875 99.0375) (end 149.1 99.025) (width 0.5) (layer "F.Cu") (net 6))
 (segment (start 149.1 99.025) (end 150.4875 99.025) (width 0.5) (layer "F.Cu") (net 6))
 (segment (start 143 97.46) (end 144.385 97.46) (width 0.5) (layer "F.Cu") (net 6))
 (segment (start 147.5 99.0375) (end 149.0875 99.0375) (width 0.5) (layer "F.Cu") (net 6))
 (segment (start 147.4375 98.975) (end 147.5 99.0375) (width 0.5) (layer "F.Cu") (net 6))
 (segment (start 144.385 97.46) (end 145.9 98.975) (width 0.5) (layer "F.Cu") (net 6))
 (segment (start 147.5 101.1625) (end 147.5 101.95) (width 0.5) (layer "F.Cu") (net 3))
 (segment (start 148.35 102.8) (end 150.1 102.8) (width 0.5) (layer "F.Cu") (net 3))
 (segment (start 150.1 102.8) (end 150.65 102.25) (width 0.5) (layer "F.Cu") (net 3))
 (segment (start 150.65 102.25) (end 150.65 101.1375) (width 0.5) (layer "F.Cu") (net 3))
 (segment (start 147.5 101.95) (end 148.35 102.8) (width 0.5) (layer "F.Cu") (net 3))
 (segment (start 150.9 95.8) (end 152.3 97.2) (width 0.25) (layer "F.Cu") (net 5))
 (segment (start 150.9 95.65) (end 150.9 95.8) (width 0.25) (layer "F.Cu") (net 5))
 (segment (start 152.3 97.2) (end 152.5 97.4) (width 0.25) (layer "F.Cu") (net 5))
 (segment (start 152.5 98.8125) (end 152.55 98.8625) (width 0.25) (layer "F.Cu") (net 5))
 (segment (start 152.5 97.4) (end 152.5 98.8125) (width 0.25) (layer "F.Cu") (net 5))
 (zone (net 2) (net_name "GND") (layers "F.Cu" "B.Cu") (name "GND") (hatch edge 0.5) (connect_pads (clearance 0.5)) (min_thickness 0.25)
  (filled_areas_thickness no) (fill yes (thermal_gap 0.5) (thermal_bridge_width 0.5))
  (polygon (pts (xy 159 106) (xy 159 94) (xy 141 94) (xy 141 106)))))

